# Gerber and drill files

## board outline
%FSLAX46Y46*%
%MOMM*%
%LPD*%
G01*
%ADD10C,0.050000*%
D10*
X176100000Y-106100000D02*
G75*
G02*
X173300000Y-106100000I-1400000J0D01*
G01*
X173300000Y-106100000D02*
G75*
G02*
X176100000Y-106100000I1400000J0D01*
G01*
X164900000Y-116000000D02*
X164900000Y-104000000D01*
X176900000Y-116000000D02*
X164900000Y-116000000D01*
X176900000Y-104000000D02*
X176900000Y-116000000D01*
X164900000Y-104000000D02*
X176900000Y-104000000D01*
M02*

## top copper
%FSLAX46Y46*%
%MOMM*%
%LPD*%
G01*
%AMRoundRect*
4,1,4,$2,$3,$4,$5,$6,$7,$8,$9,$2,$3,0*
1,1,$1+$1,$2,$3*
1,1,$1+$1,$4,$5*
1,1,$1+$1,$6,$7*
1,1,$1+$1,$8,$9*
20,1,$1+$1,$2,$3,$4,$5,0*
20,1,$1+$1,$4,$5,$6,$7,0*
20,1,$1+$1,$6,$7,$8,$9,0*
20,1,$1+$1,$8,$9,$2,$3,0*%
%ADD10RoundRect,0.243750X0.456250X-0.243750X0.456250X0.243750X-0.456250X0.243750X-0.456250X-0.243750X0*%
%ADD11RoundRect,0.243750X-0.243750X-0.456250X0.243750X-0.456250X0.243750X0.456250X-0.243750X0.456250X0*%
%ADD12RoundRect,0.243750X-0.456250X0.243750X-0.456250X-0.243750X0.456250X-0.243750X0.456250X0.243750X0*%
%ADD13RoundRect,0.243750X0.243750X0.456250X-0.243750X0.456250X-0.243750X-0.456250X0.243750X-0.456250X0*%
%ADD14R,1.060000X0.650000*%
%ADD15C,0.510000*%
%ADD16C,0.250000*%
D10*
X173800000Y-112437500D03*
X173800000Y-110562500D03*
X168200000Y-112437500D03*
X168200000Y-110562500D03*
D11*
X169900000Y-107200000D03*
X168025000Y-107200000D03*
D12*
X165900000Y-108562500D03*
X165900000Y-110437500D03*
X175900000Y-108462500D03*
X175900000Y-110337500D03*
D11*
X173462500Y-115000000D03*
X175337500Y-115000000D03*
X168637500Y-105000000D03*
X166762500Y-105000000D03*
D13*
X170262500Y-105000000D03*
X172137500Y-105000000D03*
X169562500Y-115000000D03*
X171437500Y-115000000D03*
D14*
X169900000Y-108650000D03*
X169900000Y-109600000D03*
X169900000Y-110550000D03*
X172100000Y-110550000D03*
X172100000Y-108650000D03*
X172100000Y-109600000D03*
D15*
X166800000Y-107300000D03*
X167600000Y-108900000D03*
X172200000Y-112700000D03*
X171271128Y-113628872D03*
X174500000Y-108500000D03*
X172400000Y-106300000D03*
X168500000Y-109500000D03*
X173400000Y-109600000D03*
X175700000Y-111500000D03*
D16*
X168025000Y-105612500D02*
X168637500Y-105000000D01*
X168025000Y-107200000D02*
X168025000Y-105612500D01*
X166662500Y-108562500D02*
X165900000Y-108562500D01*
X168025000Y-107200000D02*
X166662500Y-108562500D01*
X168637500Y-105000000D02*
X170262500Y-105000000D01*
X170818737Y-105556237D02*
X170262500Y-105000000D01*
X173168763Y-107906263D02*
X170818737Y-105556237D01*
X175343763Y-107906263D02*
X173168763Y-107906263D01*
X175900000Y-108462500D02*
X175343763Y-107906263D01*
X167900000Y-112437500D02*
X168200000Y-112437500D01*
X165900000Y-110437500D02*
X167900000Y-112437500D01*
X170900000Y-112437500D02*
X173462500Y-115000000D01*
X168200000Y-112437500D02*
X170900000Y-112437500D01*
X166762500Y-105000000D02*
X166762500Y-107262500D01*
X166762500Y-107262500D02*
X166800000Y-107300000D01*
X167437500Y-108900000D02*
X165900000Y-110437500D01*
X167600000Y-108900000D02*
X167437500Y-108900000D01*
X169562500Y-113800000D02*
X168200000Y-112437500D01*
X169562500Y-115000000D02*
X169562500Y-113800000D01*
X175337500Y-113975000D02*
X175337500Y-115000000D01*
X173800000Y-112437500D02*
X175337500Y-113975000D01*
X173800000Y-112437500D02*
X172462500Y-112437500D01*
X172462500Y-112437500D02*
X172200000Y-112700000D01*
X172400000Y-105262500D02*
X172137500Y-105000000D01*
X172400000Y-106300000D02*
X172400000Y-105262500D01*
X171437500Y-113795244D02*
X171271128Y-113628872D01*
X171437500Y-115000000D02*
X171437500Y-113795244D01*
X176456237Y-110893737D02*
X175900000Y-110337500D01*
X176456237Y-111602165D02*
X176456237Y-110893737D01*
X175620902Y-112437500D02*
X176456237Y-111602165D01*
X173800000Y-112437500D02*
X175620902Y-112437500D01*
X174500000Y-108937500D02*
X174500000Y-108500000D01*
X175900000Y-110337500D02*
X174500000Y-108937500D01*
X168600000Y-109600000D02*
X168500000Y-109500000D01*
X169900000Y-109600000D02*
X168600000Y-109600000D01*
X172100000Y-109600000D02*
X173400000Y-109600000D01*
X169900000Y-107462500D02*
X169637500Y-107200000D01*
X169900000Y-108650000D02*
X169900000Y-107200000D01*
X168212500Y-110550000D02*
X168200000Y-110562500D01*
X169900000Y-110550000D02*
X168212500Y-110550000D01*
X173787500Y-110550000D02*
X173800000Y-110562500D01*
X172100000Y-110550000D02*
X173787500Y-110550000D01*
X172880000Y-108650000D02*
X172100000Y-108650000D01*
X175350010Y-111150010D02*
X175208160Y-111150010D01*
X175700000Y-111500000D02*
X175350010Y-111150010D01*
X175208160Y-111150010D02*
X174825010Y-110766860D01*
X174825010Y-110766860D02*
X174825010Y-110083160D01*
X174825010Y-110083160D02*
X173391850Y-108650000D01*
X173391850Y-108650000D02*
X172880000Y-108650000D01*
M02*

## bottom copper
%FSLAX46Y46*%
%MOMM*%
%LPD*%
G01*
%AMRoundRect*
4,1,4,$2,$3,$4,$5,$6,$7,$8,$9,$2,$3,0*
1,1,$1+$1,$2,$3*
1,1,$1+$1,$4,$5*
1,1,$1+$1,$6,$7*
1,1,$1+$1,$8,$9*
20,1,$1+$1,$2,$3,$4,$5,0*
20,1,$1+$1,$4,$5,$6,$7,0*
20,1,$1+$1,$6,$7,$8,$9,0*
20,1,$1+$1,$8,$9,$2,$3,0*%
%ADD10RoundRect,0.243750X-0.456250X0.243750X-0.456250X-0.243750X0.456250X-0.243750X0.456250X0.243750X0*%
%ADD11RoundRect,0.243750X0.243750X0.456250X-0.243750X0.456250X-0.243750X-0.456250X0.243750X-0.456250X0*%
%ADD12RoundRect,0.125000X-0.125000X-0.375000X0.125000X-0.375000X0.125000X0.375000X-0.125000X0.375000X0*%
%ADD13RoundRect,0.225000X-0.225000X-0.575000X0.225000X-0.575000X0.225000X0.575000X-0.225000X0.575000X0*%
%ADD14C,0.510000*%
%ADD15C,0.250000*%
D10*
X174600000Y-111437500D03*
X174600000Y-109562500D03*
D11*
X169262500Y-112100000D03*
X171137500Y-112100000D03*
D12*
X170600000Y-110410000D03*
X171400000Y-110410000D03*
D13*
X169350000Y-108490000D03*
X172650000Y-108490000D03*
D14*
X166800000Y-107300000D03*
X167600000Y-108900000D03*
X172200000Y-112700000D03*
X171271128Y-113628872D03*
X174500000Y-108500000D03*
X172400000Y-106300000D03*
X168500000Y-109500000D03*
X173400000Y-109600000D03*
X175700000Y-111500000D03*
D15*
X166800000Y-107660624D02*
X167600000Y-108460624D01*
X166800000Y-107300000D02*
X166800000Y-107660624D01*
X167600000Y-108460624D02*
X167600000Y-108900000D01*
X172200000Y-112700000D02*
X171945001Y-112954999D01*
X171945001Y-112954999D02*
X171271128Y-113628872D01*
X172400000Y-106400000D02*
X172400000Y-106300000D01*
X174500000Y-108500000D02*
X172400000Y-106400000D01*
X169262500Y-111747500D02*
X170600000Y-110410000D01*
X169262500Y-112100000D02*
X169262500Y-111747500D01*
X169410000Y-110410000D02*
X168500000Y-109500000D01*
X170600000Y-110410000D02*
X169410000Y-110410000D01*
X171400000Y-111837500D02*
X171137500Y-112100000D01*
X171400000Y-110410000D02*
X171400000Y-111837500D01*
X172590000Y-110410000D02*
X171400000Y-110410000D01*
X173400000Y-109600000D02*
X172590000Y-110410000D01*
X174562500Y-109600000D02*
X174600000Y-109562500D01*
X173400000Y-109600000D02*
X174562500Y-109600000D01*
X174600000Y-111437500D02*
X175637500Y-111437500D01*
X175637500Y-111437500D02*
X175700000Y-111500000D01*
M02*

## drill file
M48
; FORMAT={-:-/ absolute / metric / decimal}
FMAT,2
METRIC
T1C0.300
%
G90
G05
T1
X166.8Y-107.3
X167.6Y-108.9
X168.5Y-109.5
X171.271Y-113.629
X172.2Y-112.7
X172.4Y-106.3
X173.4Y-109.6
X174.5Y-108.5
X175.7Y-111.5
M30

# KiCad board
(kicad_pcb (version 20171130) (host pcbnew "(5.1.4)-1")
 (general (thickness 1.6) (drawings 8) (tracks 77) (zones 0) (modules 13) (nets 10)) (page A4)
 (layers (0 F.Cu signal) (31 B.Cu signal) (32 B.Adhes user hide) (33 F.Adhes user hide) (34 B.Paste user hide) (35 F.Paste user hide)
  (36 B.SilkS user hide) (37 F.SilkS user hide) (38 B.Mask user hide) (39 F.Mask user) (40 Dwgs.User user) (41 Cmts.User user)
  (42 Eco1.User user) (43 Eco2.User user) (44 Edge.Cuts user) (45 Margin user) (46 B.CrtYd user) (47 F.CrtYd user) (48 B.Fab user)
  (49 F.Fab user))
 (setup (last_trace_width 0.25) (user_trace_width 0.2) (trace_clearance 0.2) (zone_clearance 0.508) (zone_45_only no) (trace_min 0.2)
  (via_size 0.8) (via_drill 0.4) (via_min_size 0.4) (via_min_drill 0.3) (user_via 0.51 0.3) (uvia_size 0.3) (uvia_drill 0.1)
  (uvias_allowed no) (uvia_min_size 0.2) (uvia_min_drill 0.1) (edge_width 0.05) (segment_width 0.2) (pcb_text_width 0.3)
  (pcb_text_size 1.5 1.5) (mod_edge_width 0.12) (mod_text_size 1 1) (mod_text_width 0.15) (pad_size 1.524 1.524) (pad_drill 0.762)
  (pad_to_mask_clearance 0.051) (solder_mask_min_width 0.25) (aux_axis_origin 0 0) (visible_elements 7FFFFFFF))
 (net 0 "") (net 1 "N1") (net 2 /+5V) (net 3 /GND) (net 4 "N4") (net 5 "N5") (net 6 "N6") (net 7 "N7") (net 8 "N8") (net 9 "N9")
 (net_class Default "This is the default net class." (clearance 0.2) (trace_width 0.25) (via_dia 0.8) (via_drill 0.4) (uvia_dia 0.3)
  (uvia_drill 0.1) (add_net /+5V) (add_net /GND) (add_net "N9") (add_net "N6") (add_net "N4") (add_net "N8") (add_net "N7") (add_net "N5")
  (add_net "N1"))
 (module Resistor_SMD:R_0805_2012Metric (layer B.Cu) (at 174.6 110.5 270)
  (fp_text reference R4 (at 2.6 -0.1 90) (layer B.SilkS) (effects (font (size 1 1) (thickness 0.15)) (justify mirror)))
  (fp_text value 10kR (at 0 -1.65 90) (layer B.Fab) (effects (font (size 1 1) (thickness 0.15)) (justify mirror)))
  (pad 2 smd roundrect (at 0.9375 0 270) (size 0.975 1.4) (layers B.Cu B.Paste B.Mask) (roundrect_rratio 0.25) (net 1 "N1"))
  (pad 1 smd roundrect (at -0.9375 0 270) (size 0.975 1.4) (layers B.Cu B.Paste B.Mask) (roundrect_rratio 0.25) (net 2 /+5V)))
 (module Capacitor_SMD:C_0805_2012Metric (layer B.Cu) (at 170.2 112.1 180)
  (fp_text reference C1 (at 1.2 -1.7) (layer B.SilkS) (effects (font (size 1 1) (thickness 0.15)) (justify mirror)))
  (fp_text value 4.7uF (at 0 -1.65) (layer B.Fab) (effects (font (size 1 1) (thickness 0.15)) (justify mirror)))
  (pad 2 smd roundrect (at 0.9375 0 180) (size 0.975 1.4) (layers B.Cu B.Paste B.Mask) (roundrect_rratio 0.25) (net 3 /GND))
  (pad 1 smd roundrect (at -0.9375 0 180) (size 0.975 1.4) (layers B.Cu B.Paste B.Mask) (roundrect_rratio 0.25) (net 2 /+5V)))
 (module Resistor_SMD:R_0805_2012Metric (layer F.Cu) (at 173.8 111.5 90)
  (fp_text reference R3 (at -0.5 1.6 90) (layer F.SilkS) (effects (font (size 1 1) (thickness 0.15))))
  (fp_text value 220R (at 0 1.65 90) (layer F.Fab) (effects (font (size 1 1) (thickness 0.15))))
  (pad 1 smd roundrect (at -0.9375 0 90) (size 0.975 1.4) (layers F.Cu F.Paste F.Mask) (roundrect_rratio 0.25) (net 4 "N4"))
  (pad 2 smd roundrect (at 0.9375 0 90) (size 0.975 1.4) (layers F.Cu F.Paste F.Mask) (roundrect_rratio 0.25) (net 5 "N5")))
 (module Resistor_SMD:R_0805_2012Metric (layer F.Cu) (at 168.2 111.5 90)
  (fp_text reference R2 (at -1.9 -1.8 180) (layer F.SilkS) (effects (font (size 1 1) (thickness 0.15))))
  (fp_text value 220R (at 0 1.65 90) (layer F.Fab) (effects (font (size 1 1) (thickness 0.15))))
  (pad 1 smd roundrect (at -0.9375 0 90) (size 0.975 1.4) (layers F.Cu F.Paste F.Mask) (roundrect_rratio 0.25) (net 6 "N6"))
  (pad 2 smd roundrect (at 0.9375 0 90) (size 0.975 1.4) (layers F.Cu F.Paste F.Mask) (roundrect_rratio 0.25) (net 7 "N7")))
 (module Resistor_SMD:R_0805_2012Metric (layer F.Cu) (at 168.9625 107.2)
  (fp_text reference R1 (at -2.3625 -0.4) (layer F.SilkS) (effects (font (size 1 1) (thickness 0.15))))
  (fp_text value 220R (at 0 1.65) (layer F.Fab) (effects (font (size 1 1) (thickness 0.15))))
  (pad 2 smd roundrect (at 0.9375 0) (size 0.975 1.4) (layers F.Cu F.Paste F.Mask) (roundrect_rratio 0.25) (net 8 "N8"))
  (pad 1 smd roundrect (at -0.9375 0) (size 0.975 1.4) (layers F.Cu F.Paste F.Mask) (roundrect_rratio 0.25) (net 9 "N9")))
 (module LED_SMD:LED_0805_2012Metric (layer F.Cu) (at 165.9 109.5 270)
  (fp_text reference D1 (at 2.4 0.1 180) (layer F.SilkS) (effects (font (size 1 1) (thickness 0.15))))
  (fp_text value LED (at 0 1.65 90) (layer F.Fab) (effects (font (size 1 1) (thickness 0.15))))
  (pad 1 smd roundrect (at -0.9375 0 270) (size 0.975 1.4) (layers F.Cu F.Paste F.Mask) (roundrect_rratio 0.25) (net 9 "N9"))
  (pad 2 smd roundrect (at 0.9375 0 270) (size 0.975 1.4) (layers F.Cu F.Paste F.Mask) (roundrect_rratio 0.25) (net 6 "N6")))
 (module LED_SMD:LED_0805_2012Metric (layer F.Cu) (at 175.9 109.4 270)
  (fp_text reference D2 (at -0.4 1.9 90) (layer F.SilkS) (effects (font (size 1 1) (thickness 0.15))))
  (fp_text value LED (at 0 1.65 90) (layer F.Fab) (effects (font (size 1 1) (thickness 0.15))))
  (pad 1 smd roundrect (at -0.9375 0 270) (size 0.975 1.4) (layers F.Cu F.Paste F.Mask) (roundrect_rratio 0.25) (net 9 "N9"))
  (pad 2 smd roundrect (at 0.9375 0 270) (size 0.975 1.4) (layers F.Cu F.Paste F.Mask) (roundrect_rratio 0.25) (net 4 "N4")))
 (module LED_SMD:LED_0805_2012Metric (layer F.Cu) (at 174.4 115)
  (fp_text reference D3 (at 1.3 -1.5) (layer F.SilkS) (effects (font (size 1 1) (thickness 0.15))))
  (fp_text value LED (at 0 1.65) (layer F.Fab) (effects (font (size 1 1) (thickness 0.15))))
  (pad 1 smd roundrect (at -0.9375 0) (size 0.975 1.4) (layers F.Cu F.Paste F.Mask) (roundrect_rratio 0.25) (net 6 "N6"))
  (pad 2 smd roundrect (at 0.9375 0) (size 0.975 1.4) (layers F.Cu F.Paste F.Mask) (roundrect_rratio 0.25) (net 4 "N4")))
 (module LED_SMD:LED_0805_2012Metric (layer F.Cu) (at 167.7 105)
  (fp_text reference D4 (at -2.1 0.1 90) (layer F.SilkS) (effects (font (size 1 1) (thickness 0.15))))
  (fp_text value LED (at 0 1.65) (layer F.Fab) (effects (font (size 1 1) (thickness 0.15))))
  (pad 2 smd roundrect (at 0.9375 0) (size 0.975 1.4) (layers F.Cu F.Paste F.Mask) (roundrect_rratio 0.25) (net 9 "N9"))
  (pad 1 smd roundrect (at -0.9375 0) (size 0.975 1.4) (layers F.Cu F.Paste F.Mask) (roundrect_rratio 0.25) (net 6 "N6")))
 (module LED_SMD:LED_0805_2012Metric (layer F.Cu) (at 171.2 105 180)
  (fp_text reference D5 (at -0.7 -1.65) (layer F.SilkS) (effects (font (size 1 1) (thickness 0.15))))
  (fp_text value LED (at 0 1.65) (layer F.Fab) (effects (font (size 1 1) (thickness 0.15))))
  (pad 2 smd roundrect (at 0.9375 0 180) (size 0.975 1.4) (layers F.Cu F.Paste F.Mask) (roundrect_rratio 0.25) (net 9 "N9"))
  (pad 1 smd roundrect (at -0.9375 0 180) (size 0.975 1.4) (layers F.Cu F.Paste F.Mask) (roundrect_rratio 0.25) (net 4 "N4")))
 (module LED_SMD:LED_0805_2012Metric (layer F.Cu) (at 170.5 115 180)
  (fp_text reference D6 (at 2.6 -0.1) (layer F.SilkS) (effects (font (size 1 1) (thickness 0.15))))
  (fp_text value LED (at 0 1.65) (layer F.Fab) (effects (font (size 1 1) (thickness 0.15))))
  (pad 2 smd roundrect (at 0.9375 0 180) (size 0.975 1.4) (layers F.Cu F.Paste F.Mask) (roundrect_rratio 0.25) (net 6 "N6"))
  (pad 1 smd roundrect (at -0.9375 0 180) (size 0.975 1.4) (layers F.Cu F.Paste F.Mask) (roundrect_rratio 0.25) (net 4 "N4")))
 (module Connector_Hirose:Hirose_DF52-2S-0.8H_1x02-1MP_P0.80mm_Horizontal (layer B.Cu) (at 171 109.3)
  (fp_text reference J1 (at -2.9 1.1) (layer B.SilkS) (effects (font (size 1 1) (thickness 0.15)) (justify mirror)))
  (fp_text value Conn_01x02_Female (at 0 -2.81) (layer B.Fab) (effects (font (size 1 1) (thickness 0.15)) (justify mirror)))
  (pad 1 smd roundrect (at -0.4 1.11) (size 0.5 1) (layers B.Cu B.Paste B.Mask) (roundrect_rratio 0.25) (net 3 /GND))
  (pad 2 smd roundrect (at 0.4 1.11) (size 0.5 1) (layers B.Cu B.Paste B.Mask) (roundrect_rratio 0.25) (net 2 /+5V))
  (pad MP smd roundrect (at -1.65 -0.81) (size 0.9 1.6) (layers B.Cu B.Paste B.Mask) (roundrect_rratio 0.25))
  (pad MP smd roundrect (at 1.65 -0.81) (size 0.9 1.6) (layers B.Cu B.Paste B.Mask) (roundrect_rratio 0.25)))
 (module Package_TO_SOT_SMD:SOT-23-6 (layer F.Cu) (at 171 109.6)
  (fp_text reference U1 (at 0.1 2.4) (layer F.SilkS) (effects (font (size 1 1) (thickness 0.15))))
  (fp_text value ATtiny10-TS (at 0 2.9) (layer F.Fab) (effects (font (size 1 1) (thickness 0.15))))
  (pad 1 smd rect (at -1.1 -0.95) (size 1.06 0.65) (layers F.Cu F.Paste F.Mask) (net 8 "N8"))
  (pad 2 smd rect (at -1.1 0) (size 1.06 0.65) (layers F.Cu F.Paste F.Mask) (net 3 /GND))
  (pad 3 smd rect (at -1.1 0.95) (size 1.06 0.65) (layers F.Cu F.Paste F.Mask) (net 7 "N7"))
  (pad 4 smd rect (at 1.1 0.95) (size 1.06 0.65) (layers F.Cu F.Paste F.Mask) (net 5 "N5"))
  (pad 6 smd rect (at 1.1 -0.95) (size 1.06 0.65) (layers F.Cu F.Paste F.Mask) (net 1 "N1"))
  (pad 5 smd rect (at 1.1 0) (size 1.06 0.65) (layers F.Cu F.Paste F.Mask) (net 2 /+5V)))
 (gr_circle (center 174.7 106.1) (end 176.1 106.1) (layer Edge.Cuts) (width 0.05))
 (gr_line (start 164.9 116) (end 164.9 104) (layer Edge.Cuts) (width 0.05))
 (gr_line (start 176.9 116) (end 164.9 116) (layer Edge.Cuts) (width 0.05))
 (gr_line (start 176.9 104) (end 176.9 116) (layer Edge.Cuts) (width 0.05))
 (gr_line (start 164.9 104) (end 176.9 104) (layer Edge.Cuts) (width 0.05))
 (segment (start 168.025 105.6125) (end 168.6375 105) (width 0.25) (layer F.Cu) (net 9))
 (segment (start 168.025 107.2) (end 168.025 105.6125) (width 0.25) (layer F.Cu) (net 9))
 (segment (start 166.6625 108.5625) (end 165.9 108.5625) (width 0.25) (layer F.Cu) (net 9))
 (segment (start 168.025 107.2) (end 166.6625 108.5625) (width 0.25) (layer F.Cu) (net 9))
 (segment (start 168.6375 105) (end 170.2625 105) (width 0.25) (layer F.Cu) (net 9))
 (segment (start 170.818737 105.556237) (end 170.2625 105) (width 0.25) (layer F.Cu) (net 9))
 (segment (start 173.168763 107.906263) (end 170.818737 105.556237) (width 0.25) (layer F.Cu) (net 9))
 (segment (start 175.343763 107.906263) (end 173.168763 107.906263) (width 0.25) (layer F.Cu) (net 9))
 (segment (start 175.9 108.4625) (end 175.343763 107.906263) (width 0.25) (layer F.Cu) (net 9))
 (segment (start 167.9 112.4375) (end 168.2 112.4375) (width 0.25) (layer F.Cu) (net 6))
 (segment (start 165.9 110.4375) (end 167.9 112.4375) (width 0.25) (layer F.Cu) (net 6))
 (segment (start 170.9 112.4375) (end 173.4625 115) (width 0.25) (layer F.Cu) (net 6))
 (segment (start 168.2 112.4375) (end 170.9 112.4375) (width 0.25) (layer F.Cu) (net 6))
 (via (at 166.8 107.3) (size 0.51) (drill 0.3) (layers F.Cu B.Cu) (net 6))
 (segment (start 166.7625 105) (end 166.7625 107.2625) (width 0.25) (layer F.Cu) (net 6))
 (segment (start 166.7625 107.2625) (end 166.8 107.3) (width 0.25) (layer F.Cu) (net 6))
 (segment (start 166.8 107.660624) (end 167.6 108.460624) (width 0.25) (layer B.Cu) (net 6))
 (segment (start 166.8 107.3) (end 166.8 107.660624) (width 0.25) (layer B.Cu) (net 6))
 (via (at 167.6 108.9) (size 0.51) (drill 0.3) (layers F.Cu B.Cu) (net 6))
 (segment (start 167.6 108.460624) (end 167.6 108.9) (width 0.25) (layer B.Cu) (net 6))
 (segment (start 167.4375 108.9) (end 165.9 110.4375) (width 0.25) (layer F.Cu) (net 6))
 (segment (start 167.6 108.9) (end 167.4375 108.9) (width 0.25) (layer F.Cu) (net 6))
 (segment (start 169.5625 113.8) (end 168.2 112.4375) (width 0.25) (layer F.Cu) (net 6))
 (segment (start 169.5625 115) (end 169.5625 113.8) (width 0.25) (layer F.Cu) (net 6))
 (segment (start 175.3375 113.975) (end 175.3375 115) (width 0.25) (layer F.Cu) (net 4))
 (segment (start 173.8 112.4375) (end 175.3375 113.975) (width 0.25) (layer F.Cu) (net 4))
 (via (at 172.2 112.7) (size 0.51) (drill 0.3) (layers F.Cu B.Cu) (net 4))
 (segment (start 173.8 112.4375) (end 172.4625 112.4375) (width 0.25) (layer F.Cu) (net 4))
 (segment (start 172.4625 112.4375) (end 172.2 112.7) (width 0.25) (layer F.Cu) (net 4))
 (segment (start 172.2 112.7) (end 171.945001 112.954999) (width 0.25) (layer B.Cu) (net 4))
 (via (at 171.271128 113.628872) (size 0.51) (drill 0.3) (layers F.Cu B.Cu) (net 4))
 (segment (start 171.945001 112.954999) (end 171.271128 113.628872) (width 0.25) (layer B.Cu) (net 4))
 (via (at 174.5 108.5) (size 0.51) (drill 0.3) (layers F.Cu B.Cu) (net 4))
 (via (at 172.4 106.3) (size 0.51) (drill 0.3) (layers F.Cu B.Cu) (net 4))
 (segment (start 172.4 105.2625) (end 172.1375 105) (width 0.25) (layer F.Cu) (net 4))
 (segment (start 172.4 106.3) (end 172.4 105.2625) (width 0.25) (layer F.Cu) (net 4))
 (segment (start 171.4375 113.795244) (end 171.271128 113.628872) (width 0.25) (layer F.Cu) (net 4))
 (segment (start 171.4375 115) (end 171.4375 113.795244) (width 0.25) (layer F.Cu) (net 4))
 (segment (start 176.456237 110.893737) (end 175.9 110.3375) (width 0.25) (layer F.Cu) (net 4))
 (segment (start 176.456237 111.602165) (end 176.456237 110.893737) (width 0.25) (layer F.Cu) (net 4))
 (segment (start 175.620902 112.4375) (end 176.456237 111.602165) (width 0.25) (layer F.Cu) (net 4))
 (segment (start 173.8 112.4375) (end 175.620902 112.4375) (width 0.25) (layer F.Cu) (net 4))
 (segment (start 174.5 108.9375) (end 174.5 108.5) (width 0.25) (layer F.Cu) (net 4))
 (segment (start 175.9 110.3375) (end 174.5 108.9375) (width 0.25) (layer F.Cu) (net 4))
 (segment (start 172.4 106.4) (end 172.4 106.3) (width 0.25) (layer B.Cu) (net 4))
 (segment (start 174.5 108.5) (end 172.4 106.4) (width 0.25) (layer B.Cu) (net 4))
 (via (at 168.5 109.5) (size 0.51) (drill 0.3) (layers F.Cu B.Cu) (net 3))
 (segment (start 169.2625 111.7475) (end 170.6 110.41) (width 0.25) (layer B.Cu) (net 3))
 (segment (start 169.2625 112.1) (end 169.2625 111.7475) (width 0.25) (layer B.Cu) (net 3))
 (segment (start 168.6 109.6) (end 168.5 109.5) (width 0.25) (layer F.Cu) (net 3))
 (segment (start 169.9 109.6) (end 168.6 109.6) (width 0.25) (layer F.Cu) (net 3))
 (segment (start 169.41 110.41) (end 168.5 109.5) (width 0.25) (layer B.Cu) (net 3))
 (segment (start 170.6 110.41) (end 169.41 110.41) (width 0.25) (layer B.Cu) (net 3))
 (via (at 173.4 109.6) (size 0.51) (drill 0.3) (layers F.Cu B.Cu) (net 2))
 (segment (start 171.4 111.8375) (end 171.1375 112.1) (width 0.25) (layer B.Cu) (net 2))
 (segment (start 171.4 110.41) (end 171.4 111.8375) (width 0.25) (layer B.Cu) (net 2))
 (segment (start 172.1 109.6) (end 173.4 109.6) (width 0.25) (layer F.Cu) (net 2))
 (segment (start 172.59 110.41) (end 171.4 110.41) (width 0.25) (layer B.Cu) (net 2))
 (segment (start 173.4 109.6) (end 172.59 110.41) (width 0.25) (layer B.Cu) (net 2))
 (segment (start 174.5625 109.6) (end 174.6 109.5625) (width 0.25) (layer B.Cu) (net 2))
 (segment (start 173.4 109.6) (end 174.5625 109.6) (width 0.25) (layer B.Cu) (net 2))
 (segment (start 169.9 107.4625) (end 169.6375 107.2) (width 0.25) (layer F.Cu) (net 8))
 (segment (start 169.9 108.65) (end 169.9 107.2) (width 0.25) (layer F.Cu) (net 8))
 (segment (start 168.2125 110.55) (end 168.2 110.5625) (width 0.25) (layer F.Cu) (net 7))
 (segment (start 169.9 110.55) (end 168.2125 110.55) (width 0.25) (layer F.Cu) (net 7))
 (segment (start 173.7875 110.55) (end 173.8 110.5625) (width 0.25) (layer F.Cu) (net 5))
 (segment (start 172.1 110.55) (end 173.7875 110.55) (width 0.25) (layer F.Cu) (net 5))
 (via (at 175.7 111.5) (size 0.51) (drill 0.3) (layers F.Cu B.Cu) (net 1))
 (segment (start 174.6 111.4375) (end 175.6375 111.4375) (width 0.25) (layer B.Cu) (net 1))
 (segment (start 175.6375 111.4375) (end 175.7 111.5) (width 0.25) (layer B.Cu) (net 1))
 (segment (start 172.88 108.65) (end 172.1 108.65) (width 0.25) (layer F.Cu) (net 1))
 (segment (start 175.35001 111.15001) (end 175.20816 111.15001) (width 0.25) (layer F.Cu) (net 1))
 (segment (start 175.7 111.5) (end 175.35001 111.15001) (width 0.25) (layer F.Cu) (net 1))
 (segment (start 175.20816 111.15001) (end 174.82501 110.76686) (width 0.25) (layer F.Cu) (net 1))
 (segment (start 174.82501 110.76686) (end 174.82501 110.08316) (width 0.25) (layer F.Cu) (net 1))
 (segment (start 174.82501 110.08316) (end 173.39185 108.65) (width 0.25) (layer F.Cu) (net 1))
 (segment (start 173.39185 108.65) (end 172.88 108.65) (width 0.25) (layer F.Cu) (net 1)))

